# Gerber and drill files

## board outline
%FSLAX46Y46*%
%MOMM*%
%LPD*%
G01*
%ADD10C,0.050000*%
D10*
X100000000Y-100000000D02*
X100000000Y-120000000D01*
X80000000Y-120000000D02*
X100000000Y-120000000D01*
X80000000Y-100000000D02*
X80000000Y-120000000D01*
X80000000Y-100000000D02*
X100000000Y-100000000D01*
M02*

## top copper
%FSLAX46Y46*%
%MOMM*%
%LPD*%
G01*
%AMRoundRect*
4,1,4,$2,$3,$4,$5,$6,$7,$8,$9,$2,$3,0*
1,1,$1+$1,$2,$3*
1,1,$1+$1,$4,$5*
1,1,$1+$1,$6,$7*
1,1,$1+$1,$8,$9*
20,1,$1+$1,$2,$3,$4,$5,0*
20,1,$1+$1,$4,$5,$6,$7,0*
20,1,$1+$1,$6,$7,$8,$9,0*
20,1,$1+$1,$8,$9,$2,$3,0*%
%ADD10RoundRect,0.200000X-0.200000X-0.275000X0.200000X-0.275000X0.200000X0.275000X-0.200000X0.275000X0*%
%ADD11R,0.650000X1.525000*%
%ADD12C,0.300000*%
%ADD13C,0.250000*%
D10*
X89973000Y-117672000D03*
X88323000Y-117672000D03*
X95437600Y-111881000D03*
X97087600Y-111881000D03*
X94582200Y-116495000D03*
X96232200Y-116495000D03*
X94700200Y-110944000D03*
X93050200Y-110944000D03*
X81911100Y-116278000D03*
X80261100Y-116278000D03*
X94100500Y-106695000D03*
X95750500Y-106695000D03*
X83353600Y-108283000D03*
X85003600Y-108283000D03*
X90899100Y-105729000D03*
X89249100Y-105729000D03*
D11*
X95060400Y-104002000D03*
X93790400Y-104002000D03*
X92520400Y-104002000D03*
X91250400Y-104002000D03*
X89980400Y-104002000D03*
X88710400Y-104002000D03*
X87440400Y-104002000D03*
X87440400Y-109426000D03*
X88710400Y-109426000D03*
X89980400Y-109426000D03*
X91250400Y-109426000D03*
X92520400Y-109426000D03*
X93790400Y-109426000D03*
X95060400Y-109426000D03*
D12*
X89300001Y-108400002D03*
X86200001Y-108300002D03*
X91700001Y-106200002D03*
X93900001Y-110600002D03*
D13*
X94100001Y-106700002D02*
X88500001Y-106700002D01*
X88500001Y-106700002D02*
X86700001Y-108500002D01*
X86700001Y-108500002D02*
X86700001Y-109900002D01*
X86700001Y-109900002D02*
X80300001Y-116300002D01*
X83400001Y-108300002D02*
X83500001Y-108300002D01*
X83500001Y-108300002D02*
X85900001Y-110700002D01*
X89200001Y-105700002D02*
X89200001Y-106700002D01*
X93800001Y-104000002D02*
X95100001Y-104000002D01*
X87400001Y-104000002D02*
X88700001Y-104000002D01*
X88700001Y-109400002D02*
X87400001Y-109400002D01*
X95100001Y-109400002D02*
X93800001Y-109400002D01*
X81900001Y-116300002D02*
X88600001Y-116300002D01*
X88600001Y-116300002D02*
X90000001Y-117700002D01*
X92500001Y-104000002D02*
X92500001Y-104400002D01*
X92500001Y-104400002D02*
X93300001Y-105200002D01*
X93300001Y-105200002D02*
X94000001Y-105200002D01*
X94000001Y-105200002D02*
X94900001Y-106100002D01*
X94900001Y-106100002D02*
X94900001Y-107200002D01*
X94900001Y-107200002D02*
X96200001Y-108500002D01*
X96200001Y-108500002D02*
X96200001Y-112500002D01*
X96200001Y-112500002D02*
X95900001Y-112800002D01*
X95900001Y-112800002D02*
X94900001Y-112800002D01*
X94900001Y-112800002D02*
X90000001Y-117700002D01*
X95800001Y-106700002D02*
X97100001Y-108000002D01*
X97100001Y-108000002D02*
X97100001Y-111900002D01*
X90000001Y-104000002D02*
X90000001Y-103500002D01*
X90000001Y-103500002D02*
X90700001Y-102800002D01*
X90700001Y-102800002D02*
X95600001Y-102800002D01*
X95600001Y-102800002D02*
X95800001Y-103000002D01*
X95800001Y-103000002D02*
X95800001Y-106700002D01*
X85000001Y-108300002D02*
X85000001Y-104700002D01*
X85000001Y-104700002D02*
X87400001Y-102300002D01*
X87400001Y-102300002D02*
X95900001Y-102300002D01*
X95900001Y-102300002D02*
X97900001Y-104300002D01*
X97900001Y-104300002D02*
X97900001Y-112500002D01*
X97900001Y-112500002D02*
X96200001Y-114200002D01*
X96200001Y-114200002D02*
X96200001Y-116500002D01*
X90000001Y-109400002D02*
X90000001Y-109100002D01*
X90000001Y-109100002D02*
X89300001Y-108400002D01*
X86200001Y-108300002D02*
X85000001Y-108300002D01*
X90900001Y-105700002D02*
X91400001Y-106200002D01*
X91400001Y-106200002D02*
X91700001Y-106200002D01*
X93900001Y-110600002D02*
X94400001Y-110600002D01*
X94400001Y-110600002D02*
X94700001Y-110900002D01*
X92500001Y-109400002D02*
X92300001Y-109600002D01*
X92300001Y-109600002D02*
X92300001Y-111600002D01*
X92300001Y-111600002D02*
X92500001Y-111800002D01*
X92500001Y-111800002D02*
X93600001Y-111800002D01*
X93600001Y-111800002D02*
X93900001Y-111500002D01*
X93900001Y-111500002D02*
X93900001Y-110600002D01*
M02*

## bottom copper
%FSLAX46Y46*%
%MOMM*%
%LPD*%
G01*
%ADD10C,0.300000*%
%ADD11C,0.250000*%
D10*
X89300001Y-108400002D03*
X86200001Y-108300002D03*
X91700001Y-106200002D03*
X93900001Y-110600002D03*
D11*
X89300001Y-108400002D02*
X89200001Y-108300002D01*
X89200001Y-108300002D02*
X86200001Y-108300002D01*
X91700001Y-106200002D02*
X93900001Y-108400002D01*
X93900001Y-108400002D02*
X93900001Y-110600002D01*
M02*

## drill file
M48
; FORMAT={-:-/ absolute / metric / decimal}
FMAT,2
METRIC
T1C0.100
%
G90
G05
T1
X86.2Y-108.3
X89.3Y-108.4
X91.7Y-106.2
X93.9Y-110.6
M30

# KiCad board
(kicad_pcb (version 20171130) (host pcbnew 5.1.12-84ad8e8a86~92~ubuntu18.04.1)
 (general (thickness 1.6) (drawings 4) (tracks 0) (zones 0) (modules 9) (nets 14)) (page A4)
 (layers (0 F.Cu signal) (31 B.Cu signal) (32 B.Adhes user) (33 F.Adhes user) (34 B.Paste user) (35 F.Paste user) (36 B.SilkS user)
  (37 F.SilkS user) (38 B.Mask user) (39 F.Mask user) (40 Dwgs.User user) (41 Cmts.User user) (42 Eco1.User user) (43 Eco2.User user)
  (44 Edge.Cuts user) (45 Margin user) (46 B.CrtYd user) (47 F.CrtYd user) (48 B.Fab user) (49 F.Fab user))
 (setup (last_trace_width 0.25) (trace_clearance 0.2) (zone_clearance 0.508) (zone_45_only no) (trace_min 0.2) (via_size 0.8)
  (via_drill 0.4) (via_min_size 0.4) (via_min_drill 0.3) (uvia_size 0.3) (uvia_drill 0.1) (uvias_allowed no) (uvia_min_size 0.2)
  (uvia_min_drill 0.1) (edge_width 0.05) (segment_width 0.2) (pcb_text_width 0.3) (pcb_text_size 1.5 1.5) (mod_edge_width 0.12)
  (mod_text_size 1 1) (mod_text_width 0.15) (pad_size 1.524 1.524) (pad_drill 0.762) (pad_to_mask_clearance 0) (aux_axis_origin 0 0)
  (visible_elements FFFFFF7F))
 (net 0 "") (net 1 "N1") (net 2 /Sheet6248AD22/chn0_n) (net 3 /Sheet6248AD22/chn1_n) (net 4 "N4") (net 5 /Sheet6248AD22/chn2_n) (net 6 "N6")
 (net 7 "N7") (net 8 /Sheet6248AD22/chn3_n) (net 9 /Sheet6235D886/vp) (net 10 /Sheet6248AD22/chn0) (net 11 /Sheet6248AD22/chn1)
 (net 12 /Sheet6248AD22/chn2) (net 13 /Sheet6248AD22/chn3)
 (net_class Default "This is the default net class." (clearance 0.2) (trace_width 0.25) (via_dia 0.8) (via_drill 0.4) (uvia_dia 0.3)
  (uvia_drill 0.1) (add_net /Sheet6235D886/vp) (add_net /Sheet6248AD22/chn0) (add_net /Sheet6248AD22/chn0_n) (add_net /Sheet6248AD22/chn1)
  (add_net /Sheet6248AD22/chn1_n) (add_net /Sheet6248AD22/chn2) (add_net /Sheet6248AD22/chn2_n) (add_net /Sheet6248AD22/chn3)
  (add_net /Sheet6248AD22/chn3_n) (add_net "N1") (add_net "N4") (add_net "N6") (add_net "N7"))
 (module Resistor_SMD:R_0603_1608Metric (layer F.Cu) (at 89.148000 117.672000)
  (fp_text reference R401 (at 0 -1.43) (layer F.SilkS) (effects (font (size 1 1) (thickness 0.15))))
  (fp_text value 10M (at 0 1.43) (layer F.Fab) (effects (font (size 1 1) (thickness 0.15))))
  (pad 2 smd roundrect (at 0.825 0) (size 0.8 0.95) (layers F.Cu F.Mask F.Paste) (roundrect_rratio 0.25) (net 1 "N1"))
  (pad 1 smd roundrect (at -0.825 0) (size 0.8 0.95) (layers F.Cu F.Mask F.Paste) (roundrect_rratio 0.25) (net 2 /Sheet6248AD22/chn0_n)))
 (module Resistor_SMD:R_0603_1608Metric (layer F.Cu) (at 96.262600 111.881000)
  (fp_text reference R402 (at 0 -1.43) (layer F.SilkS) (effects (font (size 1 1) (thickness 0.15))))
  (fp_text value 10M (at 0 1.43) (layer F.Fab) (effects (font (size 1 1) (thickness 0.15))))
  (pad 1 smd roundrect (at -0.825 0) (size 0.8 0.95) (layers F.Cu F.Mask F.Paste) (roundrect_rratio 0.25) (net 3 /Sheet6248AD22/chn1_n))
  (pad 2 smd roundrect (at 0.825 0) (size 0.8 0.95) (layers F.Cu F.Mask F.Paste) (roundrect_rratio 0.25) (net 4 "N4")))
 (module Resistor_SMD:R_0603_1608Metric (layer F.Cu) (at 95.407200 116.495000)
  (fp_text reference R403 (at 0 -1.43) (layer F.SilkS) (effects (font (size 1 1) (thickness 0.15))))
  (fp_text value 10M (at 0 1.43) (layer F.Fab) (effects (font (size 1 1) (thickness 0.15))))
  (pad 1 smd roundrect (at -0.825 0) (size 0.8 0.95) (layers F.Cu F.Mask F.Paste) (roundrect_rratio 0.25) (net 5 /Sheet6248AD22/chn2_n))
  (pad 2 smd roundrect (at 0.825 0) (size 0.8 0.95) (layers F.Cu F.Mask F.Paste) (roundrect_rratio 0.25) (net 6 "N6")))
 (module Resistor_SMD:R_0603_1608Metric (layer F.Cu) (at 93.875200 110.944000)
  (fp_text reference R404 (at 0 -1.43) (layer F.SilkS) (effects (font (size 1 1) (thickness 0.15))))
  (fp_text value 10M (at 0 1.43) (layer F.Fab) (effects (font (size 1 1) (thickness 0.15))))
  (pad 2 smd roundrect (at 0.825 0) (size 0.8 0.95) (layers F.Cu F.Mask F.Paste) (roundrect_rratio 0.25) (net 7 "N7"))
  (pad 1 smd roundrect (at -0.825 0) (size 0.8 0.95) (layers F.Cu F.Mask F.Paste) (roundrect_rratio 0.25) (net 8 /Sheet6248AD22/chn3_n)))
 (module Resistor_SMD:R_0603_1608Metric (layer F.Cu) (at 81.086100 116.278000)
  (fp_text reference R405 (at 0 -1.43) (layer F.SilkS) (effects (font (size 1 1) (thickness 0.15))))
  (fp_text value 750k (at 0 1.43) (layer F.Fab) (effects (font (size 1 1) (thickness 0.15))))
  (pad 2 smd roundrect (at 0.825 0) (size 0.8 0.95) (layers F.Cu F.Mask F.Paste) (roundrect_rratio 0.25) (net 1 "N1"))
  (pad 1 smd roundrect (at -0.825 0) (size 0.8 0.95) (layers F.Cu F.Mask F.Paste) (roundrect_rratio 0.25) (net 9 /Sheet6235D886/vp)))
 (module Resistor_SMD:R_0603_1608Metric (layer F.Cu) (at 94.925500 106.695000)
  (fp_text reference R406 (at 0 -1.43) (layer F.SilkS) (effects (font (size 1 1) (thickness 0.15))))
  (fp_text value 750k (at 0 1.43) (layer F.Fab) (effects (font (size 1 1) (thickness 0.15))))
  (pad 1 smd roundrect (at -0.825 0) (size 0.8 0.95) (layers F.Cu F.Mask F.Paste) (roundrect_rratio 0.25) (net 9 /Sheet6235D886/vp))
  (pad 2 smd roundrect (at 0.825 0) (size 0.8 0.95) (layers F.Cu F.Mask F.Paste) (roundrect_rratio 0.25) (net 4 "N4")))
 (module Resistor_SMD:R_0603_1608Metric (layer F.Cu) (at 84.178600 108.283000)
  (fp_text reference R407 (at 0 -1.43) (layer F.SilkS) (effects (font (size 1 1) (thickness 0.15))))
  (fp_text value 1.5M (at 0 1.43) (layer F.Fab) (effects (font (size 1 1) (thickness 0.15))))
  (pad 1 smd roundrect (at -0.825 0) (size 0.8 0.95) (layers F.Cu F.Mask F.Paste) (roundrect_rratio 0.25) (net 9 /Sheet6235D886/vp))
  (pad 2 smd roundrect (at 0.825 0) (size 0.8 0.95) (layers F.Cu F.Mask F.Paste) (roundrect_rratio 0.25) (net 6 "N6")))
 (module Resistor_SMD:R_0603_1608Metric (layer F.Cu) (at 90.074100 105.729000)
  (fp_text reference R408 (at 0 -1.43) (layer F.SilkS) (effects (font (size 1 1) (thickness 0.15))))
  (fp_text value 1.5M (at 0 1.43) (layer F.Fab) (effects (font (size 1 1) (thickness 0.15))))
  (pad 2 smd roundrect (at 0.825 0) (size 0.8 0.95) (layers F.Cu F.Mask F.Paste) (roundrect_rratio 0.25) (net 7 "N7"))
  (pad 1 smd roundrect (at -0.825 0) (size 0.8 0.95) (layers F.Cu F.Mask F.Paste) (roundrect_rratio 0.25) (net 9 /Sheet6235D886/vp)))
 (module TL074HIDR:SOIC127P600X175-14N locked (layer F.Cu) (at 91.250400 106.714000 270.000000)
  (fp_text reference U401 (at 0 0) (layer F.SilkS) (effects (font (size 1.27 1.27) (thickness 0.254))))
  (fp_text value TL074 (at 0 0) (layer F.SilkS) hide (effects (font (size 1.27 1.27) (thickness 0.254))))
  (pad 1 smd rect (at -2.712 -3.81) (size 0.65 1.525) (layers F.Cu F.Mask F.Paste) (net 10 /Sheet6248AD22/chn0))
  (pad 2 smd rect (at -2.712 -2.54) (size 0.65 1.525) (layers F.Cu F.Mask F.Paste) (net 10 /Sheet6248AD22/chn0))
  (pad 3 smd rect (at -2.712 -1.27) (size 0.65 1.525) (layers F.Cu F.Mask F.Paste) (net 1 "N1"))
  (pad 4 smd rect (at -2.712 0) (size 0.65 1.525) (layers F.Cu F.Mask F.Paste))
  (pad 5 smd rect (at -2.712 1.27) (size 0.65 1.525) (layers F.Cu F.Mask F.Paste) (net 4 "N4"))
  (pad 6 smd rect (at -2.712 2.54) (size 0.65 1.525) (layers F.Cu F.Mask F.Paste) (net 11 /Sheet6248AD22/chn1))
  (pad 7 smd rect (at -2.712 3.81) (size 0.65 1.525) (layers F.Cu F.Mask F.Paste) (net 11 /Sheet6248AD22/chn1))
  (pad 8 smd rect (at 2.712 3.81) (size 0.65 1.525) (layers F.Cu F.Mask F.Paste) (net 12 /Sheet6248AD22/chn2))
  (pad 9 smd rect (at 2.712 2.54) (size 0.65 1.525) (layers F.Cu F.Mask F.Paste) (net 12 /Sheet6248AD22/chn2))
  (pad 10 smd rect (at 2.712 1.27) (size 0.65 1.525) (layers F.Cu F.Mask F.Paste) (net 6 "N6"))
  (pad 11 smd rect (at 2.712 0) (size 0.65 1.525) (layers F.Cu F.Mask F.Paste))
  (pad 12 smd rect (at 2.712 -1.27) (size 0.65 1.525) (layers F.Cu F.Mask F.Paste) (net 7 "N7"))
  (pad 13 smd rect (at 2.712 -2.54) (size 0.65 1.525) (layers F.Cu F.Mask F.Paste) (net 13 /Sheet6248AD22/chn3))
  (pad 14 smd rect (at 2.712 -3.81) (size 0.65 1.525) (layers F.Cu F.Mask F.Paste) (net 13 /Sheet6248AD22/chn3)))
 (gr_line (start 100 100) (end 100 120) (layer Edge.Cuts) (width 0.05))
 (gr_line (start 80 120) (end 100 120) (layer Edge.Cuts) (width 0.05))
 (gr_line (start 80 100) (end 80 120) (layer Edge.Cuts) (width 0.05))
 (gr_line (start 80 100) (end 100 100) (layer Edge.Cuts) (width 0.05))
 (segment (start 94.100001 106.700002) (end 88.500001 106.700002) (width 0.250000) (layer F.Cu) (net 9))
 (segment (start 88.500001 106.700002) (end 86.700001 108.500002) (width 0.250000) (layer F.Cu) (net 9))
 (segment (start 86.700001 108.500002) (end 86.700001 109.900002) (width 0.250000) (layer F.Cu) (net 9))
 (segment (start 86.700001 109.900002) (end 80.300001 116.300002) (width 0.250000) (layer F.Cu) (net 9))
 (segment (start 83.400001 108.300002) (end 83.500001 108.300002) (width 0.250000) (layer F.Cu) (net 9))
 (segment (start 83.500001 108.300002) (end 85.900001 110.700002) (width 0.250000) (layer F.Cu) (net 9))
 (segment (start 89.200001 105.700002) (end 89.200001 106.700002) (width 0.250000) (layer F.Cu) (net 9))
 (segment (start 93.800001 104.000002) (end 95.100001 104.000002) (width 0.250000) (layer F.Cu) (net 10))
 (segment (start 87.400001 104.000002) (end 88.700001 104.000002) (width 0.250000) (layer F.Cu) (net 11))
 (segment (start 88.700001 109.400002) (end 87.400001 109.400002) (width 0.250000) (layer F.Cu) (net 12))
 (segment (start 95.100001 109.400002) (end 93.800001 109.400002) (width 0.250000) (layer F.Cu) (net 13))
 (segment (start 81.900001 116.300002) (end 88.600001 116.300002) (width 0.250000) (layer F.Cu) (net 1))
 (segment (start 88.600001 116.300002) (end 90.000001 117.700002) (width 0.250000) (layer F.Cu) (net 1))
 (segment (start 92.500001 104.000002) (end 92.500001 104.400002) (width 0.250000) (layer F.Cu) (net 1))
 (segment (start 92.500001 104.400002) (end 93.300001 105.200002) (width 0.250000) (layer F.Cu) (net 1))
 (segment (start 93.300001 105.200002) (end 94.000001 105.200002) (width 0.250000) (layer F.Cu) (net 1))
 (segment (start 94.000001 105.200002) (end 94.900001 106.100002) (width 0.250000) (layer F.Cu) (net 1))
 (segment (start 94.900001 106.100002) (end 94.900001 107.200002) (width 0.250000) (layer F.Cu) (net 1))
 (segment (start 94.900001 107.200002) (end 96.200001 108.500002) (width 0.250000) (layer F.Cu) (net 1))
 (segment (start 96.200001 108.500002) (end 96.200001 112.500002) (width 0.250000) (layer F.Cu) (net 1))
 (segment (start 96.200001 112.500002) (end 95.900001 112.800002) (width 0.250000) (layer F.Cu) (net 1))
 (segment (start 95.900001 112.800002) (end 94.900001 112.800002) (width 0.250000) (layer F.Cu) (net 1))
 (segment (start 94.900001 112.800002) (end 90.000001 117.700002) (width 0.250000) (layer F.Cu) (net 1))
 (segment (start 95.800001 106.700002) (end 97.100001 108.000002) (width 0.250000) (layer F.Cu) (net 4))
 (segment (start 97.100001 108.000002) (end 97.100001 111.900002) (width 0.250000) (layer F.Cu) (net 4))
 (segment (start 90.000001 104.000002) (end 90.000001 103.500002) (width 0.250000) (layer F.Cu) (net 4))
 (segment (start 90.000001 103.500002) (end 90.700001 102.800002) (width 0.250000) (layer F.Cu) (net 4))
 (segment (start 90.700001 102.800002) (end 95.600001 102.800002) (width 0.250000) (layer F.Cu) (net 4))
 (segment (start 95.600001 102.800002) (end 95.800001 103.000002) (width 0.250000) (layer F.Cu) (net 4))
 (segment (start 95.800001 103.000002) (end 95.800001 106.700002) (width 0.250000) (layer F.Cu) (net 4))
 (segment (start 85.000001 108.300002) (end 85.000001 104.700002) (width 0.250000) (layer F.Cu) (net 6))
 (segment (start 85.000001 104.700002) (end 87.400001 102.300002) (width 0.250000) (layer F.Cu) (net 6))
 (segment (start 87.400001 102.300002) (end 95.900001 102.300002) (width 0.250000) (layer F.Cu) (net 6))
 (segment (start 95.900001 102.300002) (end 97.900001 104.300002) (width 0.250000) (layer F.Cu) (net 6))
 (segment (start 97.900001 104.300002) (end 97.900001 112.500002) (width 0.250000) (layer F.Cu) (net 6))
 (segment (start 97.900001 112.500002) (end 96.200001 114.200002) (width 0.250000) (layer F.Cu) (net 6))
 (segment (start 96.200001 114.200002) (end 96.200001 116.500002) (width 0.250000) (layer F.Cu) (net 6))
 (segment (start 90.000001 109.400002) (end 90.000001 109.100002) (width 0.250000) (layer F.Cu) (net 6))
 (segment (start 90.000001 109.100002) (end 89.300001 108.400002) (width 0.250000) (layer F.Cu) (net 6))
 (segment (start 89.300001 108.400002) (end 89.200001 108.300002) (width 0.250000) (layer B.Cu) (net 6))
 (segment (start 89.200001 108.300002) (end 86.200001 108.300002) (width 0.250000) (layer B.Cu) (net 6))
 (segment (start 86.200001 108.300002) (end 85.000001 108.300002) (width 0.250000) (layer F.Cu) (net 6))
 (via micro (at 89.300001 108.400002) (size 0.300000) (drill 0.100000) (layers F.Cu B.Cu) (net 6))
 (via micro (at 86.200001 108.300002) (size 0.300000) (drill 0.100000) (layers F.Cu B.Cu) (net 6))
 (segment (start 90.900001 105.700002) (end 91.400001 106.200002) (width 0.250000) (layer F.Cu) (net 7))
 (segment (start 91.400001 106.200002) (end 91.700001 106.200002) (width 0.250000) (layer F.Cu) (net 7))
 (segment (start 91.700001 106.200002) (end 93.900001 108.400002) (width 0.250000) (layer B.Cu) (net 7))
 (segment (start 93.900001 108.400002) (end 93.900001 110.600002) (width 0.250000) (layer B.Cu) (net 7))
 (segment (start 93.900001 110.600002) (end 94.400001 110.600002) (width 0.250000) (layer F.Cu) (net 7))
 (segment (start 94.400001 110.600002) (end 94.700001 110.900002) (width 0.250000) (layer F.Cu) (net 7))
 (segment (start 92.500001 109.400002) (end 92.300001 109.600002) (width 0.250000) (layer F.Cu) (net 7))
 (segment (start 92.300001 109.600002) (end 92.300001 111.600002) (width 0.250000) (layer F.Cu) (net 7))
 (segment (start 92.300001 111.600002) (end 92.500001 111.800002) (width 0.250000) (layer F.Cu) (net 7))
 (segment (start 92.500001 111.800002) (end 93.600001 111.800002) (width 0.250000) (layer F.Cu) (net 7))
 (segment (start 93.600001 111.800002) (end 93.900001 111.500002) (width 0.250000) (layer F.Cu) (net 7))
 (segment (start 93.900001 111.500002) (end 93.900001 110.600002) (width 0.250000) (layer F.Cu) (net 7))
 (via micro (at 91.700001 106.200002) (size 0.300000) (drill 0.100000) (layers F.Cu B.Cu) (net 7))
 (via micro (at 93.900001 110.600002) (size 0.300000) (drill 0.100000) (layers F.Cu B.Cu) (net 7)))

